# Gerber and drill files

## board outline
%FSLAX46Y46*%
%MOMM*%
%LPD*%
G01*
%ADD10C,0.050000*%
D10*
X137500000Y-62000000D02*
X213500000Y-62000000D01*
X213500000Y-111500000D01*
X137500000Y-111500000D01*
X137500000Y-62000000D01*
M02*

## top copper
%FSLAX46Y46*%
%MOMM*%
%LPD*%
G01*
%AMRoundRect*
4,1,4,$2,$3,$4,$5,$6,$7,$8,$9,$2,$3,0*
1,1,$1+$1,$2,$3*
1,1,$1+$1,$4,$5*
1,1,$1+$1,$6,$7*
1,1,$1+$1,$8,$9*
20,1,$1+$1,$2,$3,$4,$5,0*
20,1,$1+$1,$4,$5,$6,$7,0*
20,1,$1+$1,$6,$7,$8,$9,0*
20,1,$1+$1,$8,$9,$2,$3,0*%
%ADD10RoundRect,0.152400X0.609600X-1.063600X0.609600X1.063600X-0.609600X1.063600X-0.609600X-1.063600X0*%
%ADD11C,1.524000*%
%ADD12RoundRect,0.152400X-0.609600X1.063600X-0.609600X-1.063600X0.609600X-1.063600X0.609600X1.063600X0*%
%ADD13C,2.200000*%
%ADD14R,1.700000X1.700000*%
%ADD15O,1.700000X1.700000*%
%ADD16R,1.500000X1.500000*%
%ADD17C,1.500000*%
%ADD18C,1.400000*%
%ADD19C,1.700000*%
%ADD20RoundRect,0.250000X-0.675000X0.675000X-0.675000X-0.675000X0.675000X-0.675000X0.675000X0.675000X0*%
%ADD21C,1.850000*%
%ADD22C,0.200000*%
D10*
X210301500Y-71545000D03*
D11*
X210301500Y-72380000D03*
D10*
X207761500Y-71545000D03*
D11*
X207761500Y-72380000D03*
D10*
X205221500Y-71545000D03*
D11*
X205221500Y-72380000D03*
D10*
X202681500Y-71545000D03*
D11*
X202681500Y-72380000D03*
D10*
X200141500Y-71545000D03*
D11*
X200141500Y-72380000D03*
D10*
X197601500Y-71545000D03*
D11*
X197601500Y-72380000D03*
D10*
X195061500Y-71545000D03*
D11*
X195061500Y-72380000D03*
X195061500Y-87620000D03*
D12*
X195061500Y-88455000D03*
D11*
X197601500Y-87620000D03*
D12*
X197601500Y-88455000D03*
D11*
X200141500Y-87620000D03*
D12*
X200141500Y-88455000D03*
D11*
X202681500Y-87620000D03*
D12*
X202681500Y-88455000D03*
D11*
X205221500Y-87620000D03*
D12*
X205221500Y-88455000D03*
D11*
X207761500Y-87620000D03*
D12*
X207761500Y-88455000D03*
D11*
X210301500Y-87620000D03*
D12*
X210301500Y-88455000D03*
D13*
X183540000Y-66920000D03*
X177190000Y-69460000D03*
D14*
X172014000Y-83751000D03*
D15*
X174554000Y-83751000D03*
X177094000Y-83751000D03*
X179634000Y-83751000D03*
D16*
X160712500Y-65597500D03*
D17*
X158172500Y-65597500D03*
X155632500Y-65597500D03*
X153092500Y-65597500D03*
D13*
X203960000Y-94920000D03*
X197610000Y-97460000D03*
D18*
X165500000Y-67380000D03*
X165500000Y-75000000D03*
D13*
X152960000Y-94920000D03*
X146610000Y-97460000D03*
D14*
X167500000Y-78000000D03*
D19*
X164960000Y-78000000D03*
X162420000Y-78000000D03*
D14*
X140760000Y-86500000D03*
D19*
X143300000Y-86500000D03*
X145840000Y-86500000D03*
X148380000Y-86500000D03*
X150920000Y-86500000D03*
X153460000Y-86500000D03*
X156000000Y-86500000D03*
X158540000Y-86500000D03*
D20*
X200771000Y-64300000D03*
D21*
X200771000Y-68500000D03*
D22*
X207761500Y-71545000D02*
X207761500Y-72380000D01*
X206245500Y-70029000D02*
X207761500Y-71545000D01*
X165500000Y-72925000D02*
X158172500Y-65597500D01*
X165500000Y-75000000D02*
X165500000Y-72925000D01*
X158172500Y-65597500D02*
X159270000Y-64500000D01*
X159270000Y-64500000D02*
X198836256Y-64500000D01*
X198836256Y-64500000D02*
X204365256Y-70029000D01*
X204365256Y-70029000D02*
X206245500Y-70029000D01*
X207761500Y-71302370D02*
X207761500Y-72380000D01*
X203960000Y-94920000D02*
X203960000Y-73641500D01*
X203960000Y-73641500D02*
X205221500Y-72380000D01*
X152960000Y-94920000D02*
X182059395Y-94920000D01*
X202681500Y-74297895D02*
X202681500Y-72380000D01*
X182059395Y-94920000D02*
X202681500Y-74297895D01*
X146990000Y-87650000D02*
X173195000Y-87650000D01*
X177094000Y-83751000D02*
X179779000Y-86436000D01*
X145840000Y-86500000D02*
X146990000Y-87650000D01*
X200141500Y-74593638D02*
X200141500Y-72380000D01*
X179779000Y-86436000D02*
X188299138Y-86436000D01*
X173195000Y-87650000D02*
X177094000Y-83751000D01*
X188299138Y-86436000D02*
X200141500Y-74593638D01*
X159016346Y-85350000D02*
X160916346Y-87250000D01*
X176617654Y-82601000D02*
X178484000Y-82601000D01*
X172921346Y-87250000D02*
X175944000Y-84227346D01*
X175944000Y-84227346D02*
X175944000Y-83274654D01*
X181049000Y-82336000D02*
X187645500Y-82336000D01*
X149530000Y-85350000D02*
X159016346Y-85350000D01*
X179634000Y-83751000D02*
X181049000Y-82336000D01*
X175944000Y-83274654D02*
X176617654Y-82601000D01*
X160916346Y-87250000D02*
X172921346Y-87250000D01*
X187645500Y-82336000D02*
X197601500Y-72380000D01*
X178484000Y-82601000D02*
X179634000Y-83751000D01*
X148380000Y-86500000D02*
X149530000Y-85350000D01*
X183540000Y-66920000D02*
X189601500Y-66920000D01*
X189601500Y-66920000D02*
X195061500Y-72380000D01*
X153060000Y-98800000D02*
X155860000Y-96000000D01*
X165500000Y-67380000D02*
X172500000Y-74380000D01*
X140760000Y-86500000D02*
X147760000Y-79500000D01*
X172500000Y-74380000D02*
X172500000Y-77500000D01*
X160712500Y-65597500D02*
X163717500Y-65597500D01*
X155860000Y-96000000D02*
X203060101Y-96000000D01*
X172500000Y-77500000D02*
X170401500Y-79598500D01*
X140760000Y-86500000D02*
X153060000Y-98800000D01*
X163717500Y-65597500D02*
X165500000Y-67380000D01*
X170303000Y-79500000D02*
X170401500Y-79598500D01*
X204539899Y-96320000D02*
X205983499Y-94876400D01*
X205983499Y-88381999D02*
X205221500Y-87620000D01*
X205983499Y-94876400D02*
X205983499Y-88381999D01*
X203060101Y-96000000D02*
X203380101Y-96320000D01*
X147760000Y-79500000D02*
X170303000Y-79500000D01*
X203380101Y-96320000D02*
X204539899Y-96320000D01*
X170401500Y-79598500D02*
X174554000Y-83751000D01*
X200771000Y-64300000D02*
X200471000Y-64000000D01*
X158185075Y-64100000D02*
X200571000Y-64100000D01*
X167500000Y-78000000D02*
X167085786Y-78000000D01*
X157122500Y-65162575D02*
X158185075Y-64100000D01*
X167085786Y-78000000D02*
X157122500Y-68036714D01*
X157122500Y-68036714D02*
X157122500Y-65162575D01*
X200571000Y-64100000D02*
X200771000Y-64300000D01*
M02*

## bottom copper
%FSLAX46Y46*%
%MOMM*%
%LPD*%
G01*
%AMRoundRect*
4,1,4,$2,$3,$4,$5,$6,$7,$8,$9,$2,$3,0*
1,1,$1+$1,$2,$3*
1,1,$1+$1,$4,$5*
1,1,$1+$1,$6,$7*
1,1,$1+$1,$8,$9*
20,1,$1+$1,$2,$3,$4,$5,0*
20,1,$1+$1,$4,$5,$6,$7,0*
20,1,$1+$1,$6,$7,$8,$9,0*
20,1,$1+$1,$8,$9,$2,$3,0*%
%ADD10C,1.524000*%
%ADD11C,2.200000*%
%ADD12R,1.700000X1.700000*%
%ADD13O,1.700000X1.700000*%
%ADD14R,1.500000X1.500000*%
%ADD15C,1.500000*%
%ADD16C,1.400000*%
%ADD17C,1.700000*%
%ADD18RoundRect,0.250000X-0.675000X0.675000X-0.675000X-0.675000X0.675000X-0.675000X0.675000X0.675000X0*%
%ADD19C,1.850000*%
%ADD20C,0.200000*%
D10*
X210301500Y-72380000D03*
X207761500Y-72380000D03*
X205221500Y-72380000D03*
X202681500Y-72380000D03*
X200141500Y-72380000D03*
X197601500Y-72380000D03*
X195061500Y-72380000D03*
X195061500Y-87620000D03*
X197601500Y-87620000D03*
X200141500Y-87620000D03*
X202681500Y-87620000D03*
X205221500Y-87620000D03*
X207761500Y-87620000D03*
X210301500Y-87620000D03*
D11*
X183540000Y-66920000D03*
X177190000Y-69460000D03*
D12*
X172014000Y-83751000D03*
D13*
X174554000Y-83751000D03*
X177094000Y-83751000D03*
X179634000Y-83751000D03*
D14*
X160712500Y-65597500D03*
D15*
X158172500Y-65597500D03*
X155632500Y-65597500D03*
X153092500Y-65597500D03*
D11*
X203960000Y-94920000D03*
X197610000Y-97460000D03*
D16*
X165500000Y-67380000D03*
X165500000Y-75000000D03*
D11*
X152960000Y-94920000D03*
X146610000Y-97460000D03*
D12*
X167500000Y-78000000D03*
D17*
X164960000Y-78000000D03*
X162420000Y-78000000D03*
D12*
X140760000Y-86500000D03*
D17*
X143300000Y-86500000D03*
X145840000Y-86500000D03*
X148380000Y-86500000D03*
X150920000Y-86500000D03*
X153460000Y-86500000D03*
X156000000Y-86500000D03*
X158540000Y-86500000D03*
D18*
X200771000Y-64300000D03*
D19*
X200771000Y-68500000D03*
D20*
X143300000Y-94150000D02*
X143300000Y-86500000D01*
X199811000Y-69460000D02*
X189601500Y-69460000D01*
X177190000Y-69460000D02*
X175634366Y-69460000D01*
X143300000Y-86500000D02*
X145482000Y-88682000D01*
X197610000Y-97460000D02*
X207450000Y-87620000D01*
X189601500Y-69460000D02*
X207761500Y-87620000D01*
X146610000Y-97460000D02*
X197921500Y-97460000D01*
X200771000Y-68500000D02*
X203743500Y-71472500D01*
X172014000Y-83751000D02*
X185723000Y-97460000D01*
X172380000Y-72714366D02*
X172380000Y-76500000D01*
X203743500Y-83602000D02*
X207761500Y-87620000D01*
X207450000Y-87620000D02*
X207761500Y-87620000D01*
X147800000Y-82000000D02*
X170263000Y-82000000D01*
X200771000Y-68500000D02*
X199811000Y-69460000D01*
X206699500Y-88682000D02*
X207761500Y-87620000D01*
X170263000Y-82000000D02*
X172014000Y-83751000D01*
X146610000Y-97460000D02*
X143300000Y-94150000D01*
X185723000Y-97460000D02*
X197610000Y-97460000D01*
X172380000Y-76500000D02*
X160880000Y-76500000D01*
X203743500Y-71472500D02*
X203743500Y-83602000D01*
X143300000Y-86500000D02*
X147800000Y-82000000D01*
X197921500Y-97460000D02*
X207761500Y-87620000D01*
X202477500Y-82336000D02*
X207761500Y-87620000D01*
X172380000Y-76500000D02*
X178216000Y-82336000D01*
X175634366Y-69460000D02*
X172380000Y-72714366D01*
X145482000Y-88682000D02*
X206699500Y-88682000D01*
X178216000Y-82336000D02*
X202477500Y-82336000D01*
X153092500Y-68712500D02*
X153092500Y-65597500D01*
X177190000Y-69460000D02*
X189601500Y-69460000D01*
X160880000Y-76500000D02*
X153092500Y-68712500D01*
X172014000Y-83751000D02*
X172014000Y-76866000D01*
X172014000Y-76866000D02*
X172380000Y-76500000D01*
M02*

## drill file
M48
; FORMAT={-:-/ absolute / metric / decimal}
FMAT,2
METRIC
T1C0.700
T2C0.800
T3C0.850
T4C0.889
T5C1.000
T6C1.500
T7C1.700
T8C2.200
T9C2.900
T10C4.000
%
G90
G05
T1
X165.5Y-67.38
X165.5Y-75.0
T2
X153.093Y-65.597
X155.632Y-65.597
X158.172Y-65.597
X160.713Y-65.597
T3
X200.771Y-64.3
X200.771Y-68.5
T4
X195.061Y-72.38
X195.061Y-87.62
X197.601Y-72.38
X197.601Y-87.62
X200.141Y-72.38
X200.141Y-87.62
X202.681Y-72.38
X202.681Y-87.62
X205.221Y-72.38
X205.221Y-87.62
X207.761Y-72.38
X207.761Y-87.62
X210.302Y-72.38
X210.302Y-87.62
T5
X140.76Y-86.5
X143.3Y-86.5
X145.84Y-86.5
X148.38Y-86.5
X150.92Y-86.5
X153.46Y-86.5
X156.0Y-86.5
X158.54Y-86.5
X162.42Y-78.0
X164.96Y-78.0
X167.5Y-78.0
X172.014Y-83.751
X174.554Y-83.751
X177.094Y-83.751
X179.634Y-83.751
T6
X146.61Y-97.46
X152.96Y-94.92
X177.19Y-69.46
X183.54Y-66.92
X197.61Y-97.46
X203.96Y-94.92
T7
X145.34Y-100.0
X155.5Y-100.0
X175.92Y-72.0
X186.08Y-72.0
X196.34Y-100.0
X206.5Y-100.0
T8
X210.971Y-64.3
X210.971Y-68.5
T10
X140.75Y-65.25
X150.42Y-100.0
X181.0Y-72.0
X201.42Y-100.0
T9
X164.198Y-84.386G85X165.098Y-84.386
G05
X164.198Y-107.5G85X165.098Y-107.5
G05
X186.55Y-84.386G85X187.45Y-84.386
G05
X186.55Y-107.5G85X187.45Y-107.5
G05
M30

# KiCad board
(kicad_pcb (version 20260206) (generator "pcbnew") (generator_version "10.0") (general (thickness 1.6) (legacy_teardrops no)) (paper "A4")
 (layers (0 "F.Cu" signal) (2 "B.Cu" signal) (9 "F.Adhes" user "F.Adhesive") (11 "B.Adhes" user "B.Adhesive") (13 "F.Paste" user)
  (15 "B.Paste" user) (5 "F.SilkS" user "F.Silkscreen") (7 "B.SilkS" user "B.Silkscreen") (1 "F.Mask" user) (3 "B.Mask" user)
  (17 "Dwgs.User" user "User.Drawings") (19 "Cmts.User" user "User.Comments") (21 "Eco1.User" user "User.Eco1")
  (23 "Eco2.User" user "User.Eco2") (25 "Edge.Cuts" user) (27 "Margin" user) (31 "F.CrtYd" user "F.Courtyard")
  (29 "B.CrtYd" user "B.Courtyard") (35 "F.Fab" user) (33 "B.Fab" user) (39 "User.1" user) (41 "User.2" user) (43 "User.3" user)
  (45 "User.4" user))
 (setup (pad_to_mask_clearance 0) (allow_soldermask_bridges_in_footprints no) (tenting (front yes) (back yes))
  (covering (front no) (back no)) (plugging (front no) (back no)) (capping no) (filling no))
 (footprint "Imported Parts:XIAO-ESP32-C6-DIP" (layer "F.Cu") (at 202.6815 80)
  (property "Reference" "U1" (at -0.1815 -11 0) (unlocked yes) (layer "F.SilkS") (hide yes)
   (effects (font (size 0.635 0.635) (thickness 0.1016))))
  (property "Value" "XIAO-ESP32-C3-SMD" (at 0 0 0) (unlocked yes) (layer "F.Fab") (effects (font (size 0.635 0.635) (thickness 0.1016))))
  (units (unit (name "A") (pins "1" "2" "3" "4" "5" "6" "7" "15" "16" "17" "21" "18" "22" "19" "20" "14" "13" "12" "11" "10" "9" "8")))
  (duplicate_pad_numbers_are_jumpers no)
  (pad "1" smd roundrect (at 7.62 -8.455 90) (size 2.432 1.524) (layers "F.Cu" "F.Mask") (roundrect_rratio 0.1)
   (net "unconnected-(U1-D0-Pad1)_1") (thermal_bridge_angle 45))
  (pad "1" thru_hole circle (at 7.62 -7.62 90) (size 1.524 1.524) (drill 0.889) (layers "*.Cu" "*.Mask") (remove_unused_layers no)
   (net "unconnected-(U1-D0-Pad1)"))
  (pad "2" smd roundrect (at 5.08 -8.455 90) (size 2.432 1.524) (layers "F.Cu" "F.Mask") (roundrect_rratio 0.1) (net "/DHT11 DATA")
   (thermal_bridge_angle 45))
  (pad "2" thru_hole circle (at 5.08 -7.62 90) (size 1.524 1.524) (drill 0.889) (layers "*.Cu" "*.Mask") (remove_unused_layers no)
   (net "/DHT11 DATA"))
  (pad "3" smd roundrect (at 2.54 -8.455 90) (size 2.432 1.524) (layers "F.Cu" "F.Mask") (roundrect_rratio 0.1) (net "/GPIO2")
   (thermal_bridge_angle 45))
  (pad "3" thru_hole circle (at 2.54 -7.62 90) (size 1.524 1.524) (drill 0.889) (layers "*.Cu" "*.Mask") (remove_unused_layers no)
   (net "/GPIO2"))
  (pad "4" smd roundrect (at 0 -8.455 90) (size 2.432 1.524) (layers "F.Cu" "F.Mask") (roundrect_rratio 0.1) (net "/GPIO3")
   (thermal_bridge_angle 45))
  (pad "4" thru_hole circle (at 0 -7.62 90) (size 1.524 1.524) (drill 0.889) (layers "*.Cu" "*.Mask") (remove_unused_layers no)
   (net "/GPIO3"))
  (pad "5" smd roundrect (at -2.54 -8.455 90) (size 2.432 1.524) (layers "F.Cu" "F.Mask") (roundrect_rratio 0.1) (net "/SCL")
   (thermal_bridge_angle 45))
  (pad "5" thru_hole circle (at -2.54 -7.62 90) (size 1.524 1.524) (drill 0.889) (layers "*.Cu" "*.Mask") (remove_unused_layers no)
   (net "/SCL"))
  (pad "6" smd roundrect (at -5.08 -8.455 90) (size 2.432 1.524) (layers "F.Cu" "F.Mask") (roundrect_rratio 0.1) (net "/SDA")
   (thermal_bridge_angle 45))
  (pad "6" thru_hole circle (at -5.08 -7.62 90) (size 1.524 1.524) (drill 0.889) (layers "*.Cu" "*.Mask") (remove_unused_layers no)
   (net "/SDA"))
  (pad "7" smd roundrect (at -7.62 -8.455 90) (size 2.432 1.524) (layers "F.Cu" "F.Mask") (roundrect_rratio 0.1) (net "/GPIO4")
   (thermal_bridge_angle 45))
  (pad "7" thru_hole circle (at -7.62 -7.62 90) (size 1.524 1.524) (drill 0.889) (layers "*.Cu" "*.Mask") (remove_unused_layers no)
   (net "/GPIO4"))
  (pad "8" thru_hole circle (at -7.62 7.62 270) (size 1.524 1.524) (drill 0.889) (layers "*.Cu" "*.Mask") (remove_unused_layers no)
   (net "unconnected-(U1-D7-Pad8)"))
  (pad "8" smd roundrect (at -7.62 8.455 270) (size 2.432 1.524) (layers "F.Cu" "F.Mask") (roundrect_rratio 0.1)
   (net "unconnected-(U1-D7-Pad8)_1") (thermal_bridge_angle 45))
  (pad "9" thru_hole circle (at -5.08 7.62 270) (size 1.524 1.524) (drill 0.889) (layers "*.Cu" "*.Mask") (remove_unused_layers no)
   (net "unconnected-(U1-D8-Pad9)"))
  (pad "9" smd roundrect (at -5.08 8.455 270) (size 2.432 1.524) (layers "F.Cu" "F.Mask") (roundrect_rratio 0.1)
   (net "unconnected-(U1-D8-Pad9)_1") (thermal_bridge_angle 45))
  (pad "10" thru_hole circle (at -2.54 7.62 270) (size 1.524 1.524) (drill 0.889) (layers "*.Cu" "*.Mask") (remove_unused_layers no)
   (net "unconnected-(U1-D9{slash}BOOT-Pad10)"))
  (pad "10" smd roundrect (at -2.54 8.455 270) (size 2.432 1.524) (layers "F.Cu" "F.Mask") (roundrect_rratio 0.1)
   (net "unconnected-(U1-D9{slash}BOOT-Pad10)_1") (thermal_bridge_angle 45))
  (pad "11" thru_hole circle (at 0 7.62 270) (size 1.524 1.524) (drill 0.889) (layers "*.Cu" "*.Mask") (remove_unused_layers no)
   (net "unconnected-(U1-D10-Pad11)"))
  (pad "11" smd roundrect (at 0 8.455 270) (size 2.432 1.524) (layers "F.Cu" "F.Mask") (roundrect_rratio 0.1)
   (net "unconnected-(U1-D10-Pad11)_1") (thermal_bridge_angle 45))
  (pad "12" thru_hole circle (at 2.54 7.62 270) (size 1.524 1.524) (drill 0.889) (layers "*.Cu" "*.Mask") (remove_unused_layers no)
   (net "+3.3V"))
  (pad "12" smd roundrect (at 2.54 8.455 270) (size 2.432 1.524) (layers "F.Cu" "F.Mask") (roundrect_rratio 0.1) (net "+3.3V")
   (thermal_bridge_angle 45))
  (pad "13" thru_hole circle (at 5.08 7.62 270) (size 1.524 1.524) (drill 0.889) (layers "*.Cu" "*.Mask") (remove_unused_layers no)
   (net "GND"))
  (pad "13" smd roundrect (at 5.08 8.455 270) (size 2.432 1.524) (layers "F.Cu" "F.Mask") (roundrect_rratio 0.1) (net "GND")
   (thermal_bridge_angle 45))
  (pad "14" thru_hole circle (at 7.62 7.62 270) (size 1.524 1.524) (drill 0.889) (layers "*.Cu" "*.Mask") (remove_unused_layers no)
   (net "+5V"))
  (pad "14" smd roundrect (at 7.62 8.455 270) (size 2.432 1.524) (layers "F.Cu" "F.Mask") (roundrect_rratio 0.1) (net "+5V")
   (thermal_bridge_angle 45)))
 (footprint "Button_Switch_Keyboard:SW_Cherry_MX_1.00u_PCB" (layer "F.Cu") (at 183.54 66.92)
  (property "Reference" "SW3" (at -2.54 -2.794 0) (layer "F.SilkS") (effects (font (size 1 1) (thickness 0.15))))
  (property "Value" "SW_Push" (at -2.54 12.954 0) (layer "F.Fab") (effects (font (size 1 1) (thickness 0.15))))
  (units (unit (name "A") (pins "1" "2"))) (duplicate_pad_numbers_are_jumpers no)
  (pad "" np_thru_hole circle (at -7.62 5.08) (size 1.7 1.7) (drill 1.7) (layers "*.Cu" "*.Mask"))
  (pad "" np_thru_hole circle (at -2.54 5.08) (size 4 4) (drill 4) (layers "*.Cu" "*.Mask"))
  (pad "" np_thru_hole circle (at 2.54 5.08) (size 1.7 1.7) (drill 1.7) (layers "*.Cu" "*.Mask"))
  (pad "1" thru_hole circle (at 0 0) (size 2.2 2.2) (drill 1.5) (layers "*.Cu" "*.Mask") (remove_unused_layers no) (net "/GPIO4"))
  (pad "2" thru_hole circle (at -6.35 2.54) (size 2.2 2.2) (drill 1.5) (layers "*.Cu" "*.Mask") (remove_unused_layers no) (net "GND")))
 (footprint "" (layer "F.Cu") (at 140.75 65.25)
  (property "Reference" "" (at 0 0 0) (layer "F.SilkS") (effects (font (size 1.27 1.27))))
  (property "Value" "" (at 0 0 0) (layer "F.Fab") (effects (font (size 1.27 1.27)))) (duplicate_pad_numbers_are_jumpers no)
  (pad "" np_thru_hole circle (at 0 0) (size 4 4) (drill 4) (layers "*.Cu" "*.Mask")))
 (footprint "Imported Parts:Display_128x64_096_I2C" (layer "F.Cu") (at 175.824 83.751)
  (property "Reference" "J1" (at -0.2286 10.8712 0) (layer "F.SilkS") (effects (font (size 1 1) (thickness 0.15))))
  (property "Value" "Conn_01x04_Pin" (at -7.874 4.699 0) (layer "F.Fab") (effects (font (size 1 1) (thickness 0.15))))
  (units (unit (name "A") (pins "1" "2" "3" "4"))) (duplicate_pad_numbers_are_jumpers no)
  (pad "" np_thru_hole oval (at -11.176 0.635) (size 3.8 2.9) (drill oval 3.8 2.9) (layers "*.Cu" "*.Mask"))
  (pad "" np_thru_hole oval (at -11.176 23.749) (size 3.8 2.9) (drill oval 3.8 2.9) (layers "*.Cu" "*.Mask"))
  (pad "" np_thru_hole oval (at 11.176 0.635) (size 3.8 2.9) (drill oval 3.8 2.9) (layers "*.Cu" "*.Mask"))
  (pad "" np_thru_hole oval (at 11.176 23.749) (size 3.8 2.9) (drill oval 3.8 2.9) (layers "*.Cu" "*.Mask"))
  (pad "1" thru_hole rect (at -3.81 0 90) (size 1.7 1.7) (drill 1) (layers "*.Cu" "*.Mask") (remove_unused_layers no) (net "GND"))
  (pad "2" thru_hole oval (at -1.27 0 90) (size 1.7 1.7) (drill 1) (layers "*.Cu" "*.Mask") (remove_unused_layers no) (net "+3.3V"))
  (pad "3" thru_hole oval (at 1.27 0 90) (size 1.7 1.7) (drill 1) (layers "*.Cu" "*.Mask") (remove_unused_layers no) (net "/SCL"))
  (pad "4" thru_hole oval (at 3.81 0 90) (size 1.7 1.7) (drill 1) (layers "*.Cu" "*.Mask") (remove_unused_layers no) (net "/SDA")))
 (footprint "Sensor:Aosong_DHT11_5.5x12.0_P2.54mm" (layer "F.Cu") (at 160.7125 65.5975 -90)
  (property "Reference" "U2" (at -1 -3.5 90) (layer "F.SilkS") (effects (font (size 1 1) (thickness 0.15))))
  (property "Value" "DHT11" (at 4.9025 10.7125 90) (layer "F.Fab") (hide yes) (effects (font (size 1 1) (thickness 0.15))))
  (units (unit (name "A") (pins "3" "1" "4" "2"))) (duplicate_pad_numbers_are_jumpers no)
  (pad "1" thru_hole rect (at 0 0 270) (size 1.5 1.5) (drill 0.8) (layers "*.Cu" "*.Mask") (remove_unused_layers no) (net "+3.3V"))
  (pad "2" thru_hole circle (at 0 2.54 270) (size 1.5 1.5) (drill 0.8) (layers "*.Cu" "*.Mask") (remove_unused_layers no)
   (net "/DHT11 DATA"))
  (pad "3" thru_hole circle (at 0 5.08 270) (size 1.5 1.5) (drill 0.8) (layers "*.Cu" "*.Mask") (remove_unused_layers no)
   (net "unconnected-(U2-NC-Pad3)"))
  (pad "4" thru_hole circle (at 0 7.62 270) (size 1.5 1.5) (drill 0.8) (layers "*.Cu" "*.Mask") (remove_unused_layers no) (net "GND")))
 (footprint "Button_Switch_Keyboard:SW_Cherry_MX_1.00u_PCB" (layer "F.Cu") (at 203.96 94.92)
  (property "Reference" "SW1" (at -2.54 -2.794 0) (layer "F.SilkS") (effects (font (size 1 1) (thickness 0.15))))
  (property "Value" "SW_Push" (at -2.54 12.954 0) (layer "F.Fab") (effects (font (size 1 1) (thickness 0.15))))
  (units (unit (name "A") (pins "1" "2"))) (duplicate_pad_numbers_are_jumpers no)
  (pad "" np_thru_hole circle (at -7.62 5.08) (size 1.7 1.7) (drill 1.7) (layers "*.Cu" "*.Mask"))
  (pad "" np_thru_hole circle (at -2.54 5.08) (size 4 4) (drill 4) (layers "*.Cu" "*.Mask"))
  (pad "" np_thru_hole circle (at 2.54 5.08) (size 1.7 1.7) (drill 1.7) (layers "*.Cu" "*.Mask"))
  (pad "1" thru_hole circle (at 0 0) (size 2.2 2.2) (drill 1.5) (layers "*.Cu" "*.Mask") (remove_unused_layers no) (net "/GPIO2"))
  (pad "2" thru_hole circle (at -6.35 2.54) (size 2.2 2.2) (drill 1.5) (layers "*.Cu" "*.Mask") (remove_unused_layers no) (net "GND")))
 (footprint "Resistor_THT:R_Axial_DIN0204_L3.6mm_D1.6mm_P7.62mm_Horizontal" (layer "F.Cu") (at 165.5 67.38 -90)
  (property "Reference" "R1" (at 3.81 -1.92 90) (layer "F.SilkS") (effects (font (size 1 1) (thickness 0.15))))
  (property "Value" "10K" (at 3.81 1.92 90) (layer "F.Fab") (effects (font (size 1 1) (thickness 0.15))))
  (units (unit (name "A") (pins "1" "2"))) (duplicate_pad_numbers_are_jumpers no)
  (pad "1" thru_hole circle (at 0 0 270) (size 1.4 1.4) (drill 0.7) (layers "*.Cu" "*.Mask") (remove_unused_layers no) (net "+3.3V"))
  (pad "2" thru_hole circle (at 7.62 0 270) (size 1.4 1.4) (drill 0.7) (layers "*.Cu" "*.Mask") (remove_unused_layers no)
   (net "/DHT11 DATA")))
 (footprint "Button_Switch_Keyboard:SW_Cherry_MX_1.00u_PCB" (layer "F.Cu") (at 152.96 94.92)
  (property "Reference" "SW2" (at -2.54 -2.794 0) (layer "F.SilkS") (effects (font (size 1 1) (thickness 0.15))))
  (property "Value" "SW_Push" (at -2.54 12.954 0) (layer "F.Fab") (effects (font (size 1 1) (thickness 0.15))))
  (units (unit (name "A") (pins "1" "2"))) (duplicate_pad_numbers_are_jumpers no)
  (pad "" np_thru_hole circle (at -7.62 5.08) (size 1.7 1.7) (drill 1.7) (layers "*.Cu" "*.Mask"))
  (pad "" np_thru_hole circle (at -2.54 5.08) (size 4 4) (drill 4) (layers "*.Cu" "*.Mask"))
  (pad "" np_thru_hole circle (at 2.54 5.08) (size 1.7 1.7) (drill 1.7) (layers "*.Cu" "*.Mask"))
  (pad "1" thru_hole circle (at 0 0) (size 2.2 2.2) (drill 1.5) (layers "*.Cu" "*.Mask") (remove_unused_layers no) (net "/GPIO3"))
  (pad "2" thru_hole circle (at -6.35 2.54) (size 2.2 2.2) (drill 1.5) (layers "*.Cu" "*.Mask") (remove_unused_layers no) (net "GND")))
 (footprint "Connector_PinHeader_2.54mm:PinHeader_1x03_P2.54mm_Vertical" (layer "B.Cu") (at 167.5 78 90)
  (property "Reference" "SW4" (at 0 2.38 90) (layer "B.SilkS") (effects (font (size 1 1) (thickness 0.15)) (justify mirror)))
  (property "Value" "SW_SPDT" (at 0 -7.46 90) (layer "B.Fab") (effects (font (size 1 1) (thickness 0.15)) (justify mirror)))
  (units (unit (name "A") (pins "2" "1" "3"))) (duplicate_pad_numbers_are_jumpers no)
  (pad "1" thru_hole rect (at 0 0 90) (size 1.7 1.7) (drill 1) (layers "*.Cu" "*.Mask") (remove_unused_layers no) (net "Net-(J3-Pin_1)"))
  (pad "2" thru_hole circle (at 0 -2.54 90) (size 1.7 1.7) (drill 1) (layers "*.Cu" "*.Mask") (remove_unused_layers no) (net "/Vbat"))
  (pad "3" thru_hole circle (at 0 -5.08 90) (size 1.7 1.7) (drill 1) (layers "*.Cu" "*.Mask") (remove_unused_layers no)
   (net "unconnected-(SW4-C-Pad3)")))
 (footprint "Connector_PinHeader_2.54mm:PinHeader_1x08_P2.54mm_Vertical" (layer "B.Cu") (at 140.76 86.5 -90)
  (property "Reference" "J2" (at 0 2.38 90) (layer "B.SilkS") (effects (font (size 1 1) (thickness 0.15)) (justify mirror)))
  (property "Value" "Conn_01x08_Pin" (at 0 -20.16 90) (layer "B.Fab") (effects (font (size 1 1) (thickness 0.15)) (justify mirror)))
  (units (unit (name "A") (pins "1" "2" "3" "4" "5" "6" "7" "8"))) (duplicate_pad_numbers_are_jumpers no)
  (pad "1" thru_hole rect (at 0 0 270) (size 1.7 1.7) (drill 1) (layers "*.Cu" "*.Mask") (remove_unused_layers no) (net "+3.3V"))
  (pad "2" thru_hole circle (at 0 -2.54 270) (size 1.7 1.7) (drill 1) (layers "*.Cu" "*.Mask") (remove_unused_layers no) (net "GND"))
  (pad "3" thru_hole circle (at 0 -5.08 270) (size 1.7 1.7) (drill 1) (layers "*.Cu" "*.Mask") (remove_unused_layers no) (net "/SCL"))
  (pad "4" thru_hole circle (at 0 -7.62 270) (size 1.7 1.7) (drill 1) (layers "*.Cu" "*.Mask") (remove_unused_layers no) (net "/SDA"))
  (pad "5" thru_hole circle (at 0 -10.16 270) (size 1.7 1.7) (drill 1) (layers "*.Cu" "*.Mask") (remove_unused_layers no)
   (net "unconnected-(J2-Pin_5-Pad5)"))
  (pad "6" thru_hole circle (at 0 -12.7 270) (size 1.7 1.7) (drill 1) (layers "*.Cu" "*.Mask") (remove_unused_layers no)
   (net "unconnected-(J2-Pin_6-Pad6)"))
  (pad "7" thru_hole circle (at 0 -15.24 270) (size 1.7 1.7) (drill 1) (layers "*.Cu" "*.Mask") (remove_unused_layers no)
   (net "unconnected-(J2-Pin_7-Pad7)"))
  (pad "8" thru_hole circle (at 0 -17.78 270) (size 1.7 1.7) (drill 1) (layers "*.Cu" "*.Mask") (remove_unused_layers no)
   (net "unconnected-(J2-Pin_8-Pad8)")))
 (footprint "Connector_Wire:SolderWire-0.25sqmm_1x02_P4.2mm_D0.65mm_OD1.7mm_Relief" (layer "B.Cu") (at 200.771 64.3 -90)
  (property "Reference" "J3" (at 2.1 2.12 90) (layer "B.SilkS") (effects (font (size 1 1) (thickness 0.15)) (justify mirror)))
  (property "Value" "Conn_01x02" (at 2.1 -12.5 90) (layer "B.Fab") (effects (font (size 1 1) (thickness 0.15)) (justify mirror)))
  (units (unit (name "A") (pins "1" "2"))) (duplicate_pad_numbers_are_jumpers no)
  (pad "" np_thru_hole circle (at 0 -10.2 270) (size 2.2 2.2) (drill 2.2) (layers "*.Cu" "*.Mask"))
  (pad "" np_thru_hole circle (at 4.2 -10.2 270) (size 2.2 2.2) (drill 2.2) (layers "*.Cu" "*.Mask"))
  (pad "1" thru_hole roundrect (at 0 0 270) (size 1.85 1.85) (drill 0.85) (layers "*.Cu" "*.Mask") (remove_unused_layers no)
   (roundrect_rratio 0.135135) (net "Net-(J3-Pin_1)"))
  (pad "2" thru_hole circle (at 4.2 0 270) (size 1.85 1.85) (drill 0.85) (layers "*.Cu" "*.Mask") (remove_unused_layers no) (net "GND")))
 (gr_rect (start 137.5 62) (end 213.5 111.5) (stroke (width 0.05) (type default)) (fill no) (layer "Edge.Cuts"))
 (segment (start 207.7615 71.545) (end 207.7615 72.38) (width 0.2) (layer "F.Cu") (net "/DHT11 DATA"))
 (segment (start 206.2455 70.029) (end 207.7615 71.545) (width 0.2) (layer "F.Cu") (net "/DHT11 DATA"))
 (segment (start 165.5 72.925) (end 158.1725 65.5975) (width 0.2) (layer "F.Cu") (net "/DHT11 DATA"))
 (segment (start 165.5 75) (end 165.5 72.925) (width 0.2) (layer "F.Cu") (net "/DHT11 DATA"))
 (segment (start 158.1725 65.5975) (end 159.27 64.5) (width 0.2) (layer "F.Cu") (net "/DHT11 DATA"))
 (segment (start 159.27 64.5) (end 198.836256 64.5) (width 0.2) (layer "F.Cu") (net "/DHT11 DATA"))
 (segment (start 198.836256 64.5) (end 204.365256 70.029) (width 0.2) (layer "F.Cu") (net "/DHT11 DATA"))
 (segment (start 204.365256 70.029) (end 206.2455 70.029) (width 0.2) (layer "F.Cu") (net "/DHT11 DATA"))
 (segment (start 207.7615 71.30237) (end 207.7615 72.38) (width 0.2) (layer "F.Cu") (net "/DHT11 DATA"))
 (segment (start 203.96 94.92) (end 203.96 73.6415) (width 0.2) (layer "F.Cu") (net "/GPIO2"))
 (segment (start 203.96 73.6415) (end 205.2215 72.38) (width 0.2) (layer "F.Cu") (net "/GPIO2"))
 (segment (start 152.96 94.92) (end 182.059395 94.92) (width 0.2) (layer "F.Cu") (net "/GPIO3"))
 (segment (start 202.6815 74.297895) (end 202.6815 72.38) (width 0.2) (layer "F.Cu") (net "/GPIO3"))
 (segment (start 182.059395 94.92) (end 202.6815 74.297895) (width 0.2) (layer "F.Cu") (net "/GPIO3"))
 (segment (start 146.99 87.65) (end 173.195 87.65) (width 0.2) (layer "F.Cu") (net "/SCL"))
 (segment (start 177.094 83.751) (end 179.779 86.436) (width 0.2) (layer "F.Cu") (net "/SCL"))
 (segment (start 145.84 86.5) (end 146.99 87.65) (width 0.2) (layer "F.Cu") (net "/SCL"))
 (segment (start 200.1415 74.593638) (end 200.1415 72.38) (width 0.2) (layer "F.Cu") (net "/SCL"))
 (segment (start 179.779 86.436) (end 188.299138 86.436) (width 0.2) (layer "F.Cu") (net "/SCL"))
 (segment (start 173.195 87.65) (end 177.094 83.751) (width 0.2) (layer "F.Cu") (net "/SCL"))
 (segment (start 188.299138 86.436) (end 200.1415 74.593638) (width 0.2) (layer "F.Cu") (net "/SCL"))
 (segment (start 159.016346 85.35) (end 160.916346 87.25) (width 0.2) (layer "F.Cu") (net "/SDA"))
 (segment (start 176.617654 82.601) (end 178.484 82.601) (width 0.2) (layer "F.Cu") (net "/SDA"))
 (segment (start 172.921346 87.25) (end 175.944 84.227346) (width 0.2) (layer "F.Cu") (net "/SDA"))
 (segment (start 175.944 84.227346) (end 175.944 83.274654) (width 0.2) (layer "F.Cu") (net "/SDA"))
 (segment (start 181.049 82.336) (end 187.6455 82.336) (width 0.2) (layer "F.Cu") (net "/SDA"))
 (segment (start 149.53 85.35) (end 159.016346 85.35) (width 0.2) (layer "F.Cu") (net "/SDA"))
 (segment (start 179.634 83.751) (end 181.049 82.336) (width 0.2) (layer "F.Cu") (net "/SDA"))
 (segment (start 175.944 83.274654) (end 176.617654 82.601) (width 0.2) (layer "F.Cu") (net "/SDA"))
 (segment (start 160.916346 87.25) (end 172.921346 87.25) (width 0.2) (layer "F.Cu") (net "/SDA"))
 (segment (start 187.6455 82.336) (end 197.6015 72.38) (width 0.2) (layer "F.Cu") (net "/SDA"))
 (segment (start 178.484 82.601) (end 179.634 83.751) (width 0.2) (layer "F.Cu") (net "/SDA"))
 (segment (start 148.38 86.5) (end 149.53 85.35) (width 0.2) (layer "F.Cu") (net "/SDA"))
 (segment (start 183.54 66.92) (end 189.6015 66.92) (width 0.2) (layer "F.Cu") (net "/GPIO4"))
 (segment (start 189.6015 66.92) (end 195.0615 72.38) (width 0.2) (layer "F.Cu") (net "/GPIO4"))
 (segment (start 153.06 98.8) (end 155.86 96) (width 0.2) (layer "F.Cu") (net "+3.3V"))
 (segment (start 165.5 67.38) (end 172.5 74.38) (width 0.2) (layer "F.Cu") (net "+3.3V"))
 (segment (start 140.76 86.5) (end 147.76 79.5) (width 0.2) (layer "F.Cu") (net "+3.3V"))
 (segment (start 172.5 74.38) (end 172.5 77.5) (width 0.2) (layer "F.Cu") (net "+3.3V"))
 (segment (start 160.7125 65.5975) (end 163.7175 65.5975) (width 0.2) (layer "F.Cu") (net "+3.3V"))
 (segment (start 155.86 96) (end 203.060101 96) (width 0.2) (layer "F.Cu") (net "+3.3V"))
 (segment (start 172.5 77.5) (end 170.4015 79.5985) (width 0.2) (layer "F.Cu") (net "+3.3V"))
 (segment (start 140.76 86.5) (end 153.06 98.8) (width 0.2) (layer "F.Cu") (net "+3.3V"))
 (segment (start 163.7175 65.5975) (end 165.5 67.38) (width 0.2) (layer "F.Cu") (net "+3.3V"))
 (segment (start 170.303 79.5) (end 170.4015 79.5985) (width 0.2) (layer "F.Cu") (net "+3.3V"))
 (segment (start 204.539899 96.32) (end 205.983499 94.8764) (width 0.2) (layer "F.Cu") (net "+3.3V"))
 (segment (start 205.983499 88.381999) (end 205.2215 87.62) (width 0.2) (layer "F.Cu") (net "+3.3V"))
 (segment (start 205.983499 94.8764) (end 205.983499 88.381999) (width 0.2) (layer "F.Cu") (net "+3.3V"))
 (segment (start 203.060101 96) (end 203.380101 96.32) (width 0.2) (layer "F.Cu") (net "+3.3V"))
 (segment (start 147.76 79.5) (end 170.303 79.5) (width 0.2) (layer "F.Cu") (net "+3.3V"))
 (segment (start 203.380101 96.32) (end 204.539899 96.32) (width 0.2) (layer "F.Cu") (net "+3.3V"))
 (segment (start 170.4015 79.5985) (end 174.554 83.751) (width 0.2) (layer "F.Cu") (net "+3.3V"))
 (segment (start 143.3 94.15) (end 143.3 86.5) (width 0.2) (layer "B.Cu") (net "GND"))
 (segment (start 199.811 69.46) (end 189.6015 69.46) (width 0.2) (layer "B.Cu") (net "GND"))
 (segment (start 177.19 69.46) (end 175.634366 69.46) (width 0.2) (layer "B.Cu") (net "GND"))
 (segment (start 143.3 86.5) (end 145.482 88.682) (width 0.2) (layer "B.Cu") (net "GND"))
 (segment (start 197.61 97.46) (end 207.45 87.62) (width 0.2) (layer "B.Cu") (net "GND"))
 (segment (start 189.6015 69.46) (end 207.7615 87.62) (width 0.2) (layer "B.Cu") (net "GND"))
 (segment (start 146.61 97.46) (end 197.9215 97.46) (width 0.2) (layer "B.Cu") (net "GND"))
 (segment (start 200.771 68.5) (end 203.7435 71.4725) (width 0.2) (layer "B.Cu") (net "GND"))
 (segment (start 172.014 83.751) (end 185.723 97.46) (width 0.2) (layer "B.Cu") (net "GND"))
 (segment (start 172.38 72.714366) (end 172.38 76.5) (width 0.2) (layer "B.Cu") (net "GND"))
 (segment (start 203.7435 83.602) (end 207.7615 87.62) (width 0.2) (layer "B.Cu") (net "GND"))
 (segment (start 207.45 87.62) (end 207.7615 87.62) (width 0.2) (layer "B.Cu") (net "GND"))
 (segment (start 147.8 82) (end 170.263 82) (width 0.2) (layer "B.Cu") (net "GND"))
 (segment (start 200.771 68.5) (end 199.811 69.46) (width 0.2) (layer "B.Cu") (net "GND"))
 (segment (start 206.6995 88.682) (end 207.7615 87.62) (width 0.2) (layer "B.Cu") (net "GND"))
 (segment (start 170.263 82) (end 172.014 83.751) (width 0.2) (layer "B.Cu") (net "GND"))
 (segment (start 146.61 97.46) (end 143.3 94.15) (width 0.2) (layer "B.Cu") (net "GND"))
 (segment (start 185.723 97.46) (end 197.61 97.46) (width 0.2) (layer "B.Cu") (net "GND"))
 (segment (start 172.38 76.5) (end 160.88 76.5) (width 0.2) (layer "B.Cu") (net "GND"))
 (segment (start 203.7435 71.4725) (end 203.7435 83.602) (width 0.2) (layer "B.Cu") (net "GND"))
 (segment (start 143.3 86.5) (end 147.8 82) (width 0.2) (layer "B.Cu") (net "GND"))
 (segment (start 197.9215 97.46) (end 207.7615 87.62) (width 0.2) (layer "B.Cu") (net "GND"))
 (segment (start 202.4775 82.336) (end 207.7615 87.62) (width 0.2) (layer "B.Cu") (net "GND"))
 (segment (start 172.38 76.5) (end 178.216 82.336) (width 0.2) (layer "B.Cu") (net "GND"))
 (segment (start 175.634366 69.46) (end 172.38 72.714366) (width 0.2) (layer "B.Cu") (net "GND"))
 (segment (start 145.482 88.682) (end 206.6995 88.682) (width 0.2) (layer "B.Cu") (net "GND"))
 (segment (start 178.216 82.336) (end 202.4775 82.336) (width 0.2) (layer "B.Cu") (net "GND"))
 (segment (start 153.0925 68.7125) (end 153.0925 65.5975) (width 0.2) (layer "B.Cu") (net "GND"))
 (segment (start 177.19 69.46) (end 189.6015 69.46) (width 0.2) (layer "B.Cu") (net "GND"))
 (segment (start 160.88 76.5) (end 153.0925 68.7125) (width 0.2) (layer "B.Cu") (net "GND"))
 (segment (start 172.014 83.751) (end 172.014 76.866) (width 0.2) (layer "B.Cu") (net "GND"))
 (segment (start 172.014 76.866) (end 172.38 76.5) (width 0.2) (layer "B.Cu") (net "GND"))
 (segment (start 200.771 64.3) (end 200.471 64) (width 0.2) (layer "F.Cu") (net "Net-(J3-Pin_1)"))
 (segment (start 158.185075 64.1) (end 200.571 64.1) (width 0.2) (layer "F.Cu") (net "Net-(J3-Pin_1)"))
 (segment (start 167.5 78) (end 167.085786 78) (width 0.2) (layer "F.Cu") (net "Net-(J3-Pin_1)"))
 (segment (start 157.1225 65.162575) (end 158.185075 64.1) (width 0.2) (layer "F.Cu") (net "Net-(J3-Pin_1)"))
 (segment (start 167.085786 78) (end 157.1225 68.036714) (width 0.2) (layer "F.Cu") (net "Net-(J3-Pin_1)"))
 (segment (start 157.1225 68.036714) (end 157.1225 65.162575) (width 0.2) (layer "F.Cu") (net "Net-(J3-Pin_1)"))
 (segment (start 200.571 64.1) (end 200.771 64.3) (width 0.2) (layer "F.Cu") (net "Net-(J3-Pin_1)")))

